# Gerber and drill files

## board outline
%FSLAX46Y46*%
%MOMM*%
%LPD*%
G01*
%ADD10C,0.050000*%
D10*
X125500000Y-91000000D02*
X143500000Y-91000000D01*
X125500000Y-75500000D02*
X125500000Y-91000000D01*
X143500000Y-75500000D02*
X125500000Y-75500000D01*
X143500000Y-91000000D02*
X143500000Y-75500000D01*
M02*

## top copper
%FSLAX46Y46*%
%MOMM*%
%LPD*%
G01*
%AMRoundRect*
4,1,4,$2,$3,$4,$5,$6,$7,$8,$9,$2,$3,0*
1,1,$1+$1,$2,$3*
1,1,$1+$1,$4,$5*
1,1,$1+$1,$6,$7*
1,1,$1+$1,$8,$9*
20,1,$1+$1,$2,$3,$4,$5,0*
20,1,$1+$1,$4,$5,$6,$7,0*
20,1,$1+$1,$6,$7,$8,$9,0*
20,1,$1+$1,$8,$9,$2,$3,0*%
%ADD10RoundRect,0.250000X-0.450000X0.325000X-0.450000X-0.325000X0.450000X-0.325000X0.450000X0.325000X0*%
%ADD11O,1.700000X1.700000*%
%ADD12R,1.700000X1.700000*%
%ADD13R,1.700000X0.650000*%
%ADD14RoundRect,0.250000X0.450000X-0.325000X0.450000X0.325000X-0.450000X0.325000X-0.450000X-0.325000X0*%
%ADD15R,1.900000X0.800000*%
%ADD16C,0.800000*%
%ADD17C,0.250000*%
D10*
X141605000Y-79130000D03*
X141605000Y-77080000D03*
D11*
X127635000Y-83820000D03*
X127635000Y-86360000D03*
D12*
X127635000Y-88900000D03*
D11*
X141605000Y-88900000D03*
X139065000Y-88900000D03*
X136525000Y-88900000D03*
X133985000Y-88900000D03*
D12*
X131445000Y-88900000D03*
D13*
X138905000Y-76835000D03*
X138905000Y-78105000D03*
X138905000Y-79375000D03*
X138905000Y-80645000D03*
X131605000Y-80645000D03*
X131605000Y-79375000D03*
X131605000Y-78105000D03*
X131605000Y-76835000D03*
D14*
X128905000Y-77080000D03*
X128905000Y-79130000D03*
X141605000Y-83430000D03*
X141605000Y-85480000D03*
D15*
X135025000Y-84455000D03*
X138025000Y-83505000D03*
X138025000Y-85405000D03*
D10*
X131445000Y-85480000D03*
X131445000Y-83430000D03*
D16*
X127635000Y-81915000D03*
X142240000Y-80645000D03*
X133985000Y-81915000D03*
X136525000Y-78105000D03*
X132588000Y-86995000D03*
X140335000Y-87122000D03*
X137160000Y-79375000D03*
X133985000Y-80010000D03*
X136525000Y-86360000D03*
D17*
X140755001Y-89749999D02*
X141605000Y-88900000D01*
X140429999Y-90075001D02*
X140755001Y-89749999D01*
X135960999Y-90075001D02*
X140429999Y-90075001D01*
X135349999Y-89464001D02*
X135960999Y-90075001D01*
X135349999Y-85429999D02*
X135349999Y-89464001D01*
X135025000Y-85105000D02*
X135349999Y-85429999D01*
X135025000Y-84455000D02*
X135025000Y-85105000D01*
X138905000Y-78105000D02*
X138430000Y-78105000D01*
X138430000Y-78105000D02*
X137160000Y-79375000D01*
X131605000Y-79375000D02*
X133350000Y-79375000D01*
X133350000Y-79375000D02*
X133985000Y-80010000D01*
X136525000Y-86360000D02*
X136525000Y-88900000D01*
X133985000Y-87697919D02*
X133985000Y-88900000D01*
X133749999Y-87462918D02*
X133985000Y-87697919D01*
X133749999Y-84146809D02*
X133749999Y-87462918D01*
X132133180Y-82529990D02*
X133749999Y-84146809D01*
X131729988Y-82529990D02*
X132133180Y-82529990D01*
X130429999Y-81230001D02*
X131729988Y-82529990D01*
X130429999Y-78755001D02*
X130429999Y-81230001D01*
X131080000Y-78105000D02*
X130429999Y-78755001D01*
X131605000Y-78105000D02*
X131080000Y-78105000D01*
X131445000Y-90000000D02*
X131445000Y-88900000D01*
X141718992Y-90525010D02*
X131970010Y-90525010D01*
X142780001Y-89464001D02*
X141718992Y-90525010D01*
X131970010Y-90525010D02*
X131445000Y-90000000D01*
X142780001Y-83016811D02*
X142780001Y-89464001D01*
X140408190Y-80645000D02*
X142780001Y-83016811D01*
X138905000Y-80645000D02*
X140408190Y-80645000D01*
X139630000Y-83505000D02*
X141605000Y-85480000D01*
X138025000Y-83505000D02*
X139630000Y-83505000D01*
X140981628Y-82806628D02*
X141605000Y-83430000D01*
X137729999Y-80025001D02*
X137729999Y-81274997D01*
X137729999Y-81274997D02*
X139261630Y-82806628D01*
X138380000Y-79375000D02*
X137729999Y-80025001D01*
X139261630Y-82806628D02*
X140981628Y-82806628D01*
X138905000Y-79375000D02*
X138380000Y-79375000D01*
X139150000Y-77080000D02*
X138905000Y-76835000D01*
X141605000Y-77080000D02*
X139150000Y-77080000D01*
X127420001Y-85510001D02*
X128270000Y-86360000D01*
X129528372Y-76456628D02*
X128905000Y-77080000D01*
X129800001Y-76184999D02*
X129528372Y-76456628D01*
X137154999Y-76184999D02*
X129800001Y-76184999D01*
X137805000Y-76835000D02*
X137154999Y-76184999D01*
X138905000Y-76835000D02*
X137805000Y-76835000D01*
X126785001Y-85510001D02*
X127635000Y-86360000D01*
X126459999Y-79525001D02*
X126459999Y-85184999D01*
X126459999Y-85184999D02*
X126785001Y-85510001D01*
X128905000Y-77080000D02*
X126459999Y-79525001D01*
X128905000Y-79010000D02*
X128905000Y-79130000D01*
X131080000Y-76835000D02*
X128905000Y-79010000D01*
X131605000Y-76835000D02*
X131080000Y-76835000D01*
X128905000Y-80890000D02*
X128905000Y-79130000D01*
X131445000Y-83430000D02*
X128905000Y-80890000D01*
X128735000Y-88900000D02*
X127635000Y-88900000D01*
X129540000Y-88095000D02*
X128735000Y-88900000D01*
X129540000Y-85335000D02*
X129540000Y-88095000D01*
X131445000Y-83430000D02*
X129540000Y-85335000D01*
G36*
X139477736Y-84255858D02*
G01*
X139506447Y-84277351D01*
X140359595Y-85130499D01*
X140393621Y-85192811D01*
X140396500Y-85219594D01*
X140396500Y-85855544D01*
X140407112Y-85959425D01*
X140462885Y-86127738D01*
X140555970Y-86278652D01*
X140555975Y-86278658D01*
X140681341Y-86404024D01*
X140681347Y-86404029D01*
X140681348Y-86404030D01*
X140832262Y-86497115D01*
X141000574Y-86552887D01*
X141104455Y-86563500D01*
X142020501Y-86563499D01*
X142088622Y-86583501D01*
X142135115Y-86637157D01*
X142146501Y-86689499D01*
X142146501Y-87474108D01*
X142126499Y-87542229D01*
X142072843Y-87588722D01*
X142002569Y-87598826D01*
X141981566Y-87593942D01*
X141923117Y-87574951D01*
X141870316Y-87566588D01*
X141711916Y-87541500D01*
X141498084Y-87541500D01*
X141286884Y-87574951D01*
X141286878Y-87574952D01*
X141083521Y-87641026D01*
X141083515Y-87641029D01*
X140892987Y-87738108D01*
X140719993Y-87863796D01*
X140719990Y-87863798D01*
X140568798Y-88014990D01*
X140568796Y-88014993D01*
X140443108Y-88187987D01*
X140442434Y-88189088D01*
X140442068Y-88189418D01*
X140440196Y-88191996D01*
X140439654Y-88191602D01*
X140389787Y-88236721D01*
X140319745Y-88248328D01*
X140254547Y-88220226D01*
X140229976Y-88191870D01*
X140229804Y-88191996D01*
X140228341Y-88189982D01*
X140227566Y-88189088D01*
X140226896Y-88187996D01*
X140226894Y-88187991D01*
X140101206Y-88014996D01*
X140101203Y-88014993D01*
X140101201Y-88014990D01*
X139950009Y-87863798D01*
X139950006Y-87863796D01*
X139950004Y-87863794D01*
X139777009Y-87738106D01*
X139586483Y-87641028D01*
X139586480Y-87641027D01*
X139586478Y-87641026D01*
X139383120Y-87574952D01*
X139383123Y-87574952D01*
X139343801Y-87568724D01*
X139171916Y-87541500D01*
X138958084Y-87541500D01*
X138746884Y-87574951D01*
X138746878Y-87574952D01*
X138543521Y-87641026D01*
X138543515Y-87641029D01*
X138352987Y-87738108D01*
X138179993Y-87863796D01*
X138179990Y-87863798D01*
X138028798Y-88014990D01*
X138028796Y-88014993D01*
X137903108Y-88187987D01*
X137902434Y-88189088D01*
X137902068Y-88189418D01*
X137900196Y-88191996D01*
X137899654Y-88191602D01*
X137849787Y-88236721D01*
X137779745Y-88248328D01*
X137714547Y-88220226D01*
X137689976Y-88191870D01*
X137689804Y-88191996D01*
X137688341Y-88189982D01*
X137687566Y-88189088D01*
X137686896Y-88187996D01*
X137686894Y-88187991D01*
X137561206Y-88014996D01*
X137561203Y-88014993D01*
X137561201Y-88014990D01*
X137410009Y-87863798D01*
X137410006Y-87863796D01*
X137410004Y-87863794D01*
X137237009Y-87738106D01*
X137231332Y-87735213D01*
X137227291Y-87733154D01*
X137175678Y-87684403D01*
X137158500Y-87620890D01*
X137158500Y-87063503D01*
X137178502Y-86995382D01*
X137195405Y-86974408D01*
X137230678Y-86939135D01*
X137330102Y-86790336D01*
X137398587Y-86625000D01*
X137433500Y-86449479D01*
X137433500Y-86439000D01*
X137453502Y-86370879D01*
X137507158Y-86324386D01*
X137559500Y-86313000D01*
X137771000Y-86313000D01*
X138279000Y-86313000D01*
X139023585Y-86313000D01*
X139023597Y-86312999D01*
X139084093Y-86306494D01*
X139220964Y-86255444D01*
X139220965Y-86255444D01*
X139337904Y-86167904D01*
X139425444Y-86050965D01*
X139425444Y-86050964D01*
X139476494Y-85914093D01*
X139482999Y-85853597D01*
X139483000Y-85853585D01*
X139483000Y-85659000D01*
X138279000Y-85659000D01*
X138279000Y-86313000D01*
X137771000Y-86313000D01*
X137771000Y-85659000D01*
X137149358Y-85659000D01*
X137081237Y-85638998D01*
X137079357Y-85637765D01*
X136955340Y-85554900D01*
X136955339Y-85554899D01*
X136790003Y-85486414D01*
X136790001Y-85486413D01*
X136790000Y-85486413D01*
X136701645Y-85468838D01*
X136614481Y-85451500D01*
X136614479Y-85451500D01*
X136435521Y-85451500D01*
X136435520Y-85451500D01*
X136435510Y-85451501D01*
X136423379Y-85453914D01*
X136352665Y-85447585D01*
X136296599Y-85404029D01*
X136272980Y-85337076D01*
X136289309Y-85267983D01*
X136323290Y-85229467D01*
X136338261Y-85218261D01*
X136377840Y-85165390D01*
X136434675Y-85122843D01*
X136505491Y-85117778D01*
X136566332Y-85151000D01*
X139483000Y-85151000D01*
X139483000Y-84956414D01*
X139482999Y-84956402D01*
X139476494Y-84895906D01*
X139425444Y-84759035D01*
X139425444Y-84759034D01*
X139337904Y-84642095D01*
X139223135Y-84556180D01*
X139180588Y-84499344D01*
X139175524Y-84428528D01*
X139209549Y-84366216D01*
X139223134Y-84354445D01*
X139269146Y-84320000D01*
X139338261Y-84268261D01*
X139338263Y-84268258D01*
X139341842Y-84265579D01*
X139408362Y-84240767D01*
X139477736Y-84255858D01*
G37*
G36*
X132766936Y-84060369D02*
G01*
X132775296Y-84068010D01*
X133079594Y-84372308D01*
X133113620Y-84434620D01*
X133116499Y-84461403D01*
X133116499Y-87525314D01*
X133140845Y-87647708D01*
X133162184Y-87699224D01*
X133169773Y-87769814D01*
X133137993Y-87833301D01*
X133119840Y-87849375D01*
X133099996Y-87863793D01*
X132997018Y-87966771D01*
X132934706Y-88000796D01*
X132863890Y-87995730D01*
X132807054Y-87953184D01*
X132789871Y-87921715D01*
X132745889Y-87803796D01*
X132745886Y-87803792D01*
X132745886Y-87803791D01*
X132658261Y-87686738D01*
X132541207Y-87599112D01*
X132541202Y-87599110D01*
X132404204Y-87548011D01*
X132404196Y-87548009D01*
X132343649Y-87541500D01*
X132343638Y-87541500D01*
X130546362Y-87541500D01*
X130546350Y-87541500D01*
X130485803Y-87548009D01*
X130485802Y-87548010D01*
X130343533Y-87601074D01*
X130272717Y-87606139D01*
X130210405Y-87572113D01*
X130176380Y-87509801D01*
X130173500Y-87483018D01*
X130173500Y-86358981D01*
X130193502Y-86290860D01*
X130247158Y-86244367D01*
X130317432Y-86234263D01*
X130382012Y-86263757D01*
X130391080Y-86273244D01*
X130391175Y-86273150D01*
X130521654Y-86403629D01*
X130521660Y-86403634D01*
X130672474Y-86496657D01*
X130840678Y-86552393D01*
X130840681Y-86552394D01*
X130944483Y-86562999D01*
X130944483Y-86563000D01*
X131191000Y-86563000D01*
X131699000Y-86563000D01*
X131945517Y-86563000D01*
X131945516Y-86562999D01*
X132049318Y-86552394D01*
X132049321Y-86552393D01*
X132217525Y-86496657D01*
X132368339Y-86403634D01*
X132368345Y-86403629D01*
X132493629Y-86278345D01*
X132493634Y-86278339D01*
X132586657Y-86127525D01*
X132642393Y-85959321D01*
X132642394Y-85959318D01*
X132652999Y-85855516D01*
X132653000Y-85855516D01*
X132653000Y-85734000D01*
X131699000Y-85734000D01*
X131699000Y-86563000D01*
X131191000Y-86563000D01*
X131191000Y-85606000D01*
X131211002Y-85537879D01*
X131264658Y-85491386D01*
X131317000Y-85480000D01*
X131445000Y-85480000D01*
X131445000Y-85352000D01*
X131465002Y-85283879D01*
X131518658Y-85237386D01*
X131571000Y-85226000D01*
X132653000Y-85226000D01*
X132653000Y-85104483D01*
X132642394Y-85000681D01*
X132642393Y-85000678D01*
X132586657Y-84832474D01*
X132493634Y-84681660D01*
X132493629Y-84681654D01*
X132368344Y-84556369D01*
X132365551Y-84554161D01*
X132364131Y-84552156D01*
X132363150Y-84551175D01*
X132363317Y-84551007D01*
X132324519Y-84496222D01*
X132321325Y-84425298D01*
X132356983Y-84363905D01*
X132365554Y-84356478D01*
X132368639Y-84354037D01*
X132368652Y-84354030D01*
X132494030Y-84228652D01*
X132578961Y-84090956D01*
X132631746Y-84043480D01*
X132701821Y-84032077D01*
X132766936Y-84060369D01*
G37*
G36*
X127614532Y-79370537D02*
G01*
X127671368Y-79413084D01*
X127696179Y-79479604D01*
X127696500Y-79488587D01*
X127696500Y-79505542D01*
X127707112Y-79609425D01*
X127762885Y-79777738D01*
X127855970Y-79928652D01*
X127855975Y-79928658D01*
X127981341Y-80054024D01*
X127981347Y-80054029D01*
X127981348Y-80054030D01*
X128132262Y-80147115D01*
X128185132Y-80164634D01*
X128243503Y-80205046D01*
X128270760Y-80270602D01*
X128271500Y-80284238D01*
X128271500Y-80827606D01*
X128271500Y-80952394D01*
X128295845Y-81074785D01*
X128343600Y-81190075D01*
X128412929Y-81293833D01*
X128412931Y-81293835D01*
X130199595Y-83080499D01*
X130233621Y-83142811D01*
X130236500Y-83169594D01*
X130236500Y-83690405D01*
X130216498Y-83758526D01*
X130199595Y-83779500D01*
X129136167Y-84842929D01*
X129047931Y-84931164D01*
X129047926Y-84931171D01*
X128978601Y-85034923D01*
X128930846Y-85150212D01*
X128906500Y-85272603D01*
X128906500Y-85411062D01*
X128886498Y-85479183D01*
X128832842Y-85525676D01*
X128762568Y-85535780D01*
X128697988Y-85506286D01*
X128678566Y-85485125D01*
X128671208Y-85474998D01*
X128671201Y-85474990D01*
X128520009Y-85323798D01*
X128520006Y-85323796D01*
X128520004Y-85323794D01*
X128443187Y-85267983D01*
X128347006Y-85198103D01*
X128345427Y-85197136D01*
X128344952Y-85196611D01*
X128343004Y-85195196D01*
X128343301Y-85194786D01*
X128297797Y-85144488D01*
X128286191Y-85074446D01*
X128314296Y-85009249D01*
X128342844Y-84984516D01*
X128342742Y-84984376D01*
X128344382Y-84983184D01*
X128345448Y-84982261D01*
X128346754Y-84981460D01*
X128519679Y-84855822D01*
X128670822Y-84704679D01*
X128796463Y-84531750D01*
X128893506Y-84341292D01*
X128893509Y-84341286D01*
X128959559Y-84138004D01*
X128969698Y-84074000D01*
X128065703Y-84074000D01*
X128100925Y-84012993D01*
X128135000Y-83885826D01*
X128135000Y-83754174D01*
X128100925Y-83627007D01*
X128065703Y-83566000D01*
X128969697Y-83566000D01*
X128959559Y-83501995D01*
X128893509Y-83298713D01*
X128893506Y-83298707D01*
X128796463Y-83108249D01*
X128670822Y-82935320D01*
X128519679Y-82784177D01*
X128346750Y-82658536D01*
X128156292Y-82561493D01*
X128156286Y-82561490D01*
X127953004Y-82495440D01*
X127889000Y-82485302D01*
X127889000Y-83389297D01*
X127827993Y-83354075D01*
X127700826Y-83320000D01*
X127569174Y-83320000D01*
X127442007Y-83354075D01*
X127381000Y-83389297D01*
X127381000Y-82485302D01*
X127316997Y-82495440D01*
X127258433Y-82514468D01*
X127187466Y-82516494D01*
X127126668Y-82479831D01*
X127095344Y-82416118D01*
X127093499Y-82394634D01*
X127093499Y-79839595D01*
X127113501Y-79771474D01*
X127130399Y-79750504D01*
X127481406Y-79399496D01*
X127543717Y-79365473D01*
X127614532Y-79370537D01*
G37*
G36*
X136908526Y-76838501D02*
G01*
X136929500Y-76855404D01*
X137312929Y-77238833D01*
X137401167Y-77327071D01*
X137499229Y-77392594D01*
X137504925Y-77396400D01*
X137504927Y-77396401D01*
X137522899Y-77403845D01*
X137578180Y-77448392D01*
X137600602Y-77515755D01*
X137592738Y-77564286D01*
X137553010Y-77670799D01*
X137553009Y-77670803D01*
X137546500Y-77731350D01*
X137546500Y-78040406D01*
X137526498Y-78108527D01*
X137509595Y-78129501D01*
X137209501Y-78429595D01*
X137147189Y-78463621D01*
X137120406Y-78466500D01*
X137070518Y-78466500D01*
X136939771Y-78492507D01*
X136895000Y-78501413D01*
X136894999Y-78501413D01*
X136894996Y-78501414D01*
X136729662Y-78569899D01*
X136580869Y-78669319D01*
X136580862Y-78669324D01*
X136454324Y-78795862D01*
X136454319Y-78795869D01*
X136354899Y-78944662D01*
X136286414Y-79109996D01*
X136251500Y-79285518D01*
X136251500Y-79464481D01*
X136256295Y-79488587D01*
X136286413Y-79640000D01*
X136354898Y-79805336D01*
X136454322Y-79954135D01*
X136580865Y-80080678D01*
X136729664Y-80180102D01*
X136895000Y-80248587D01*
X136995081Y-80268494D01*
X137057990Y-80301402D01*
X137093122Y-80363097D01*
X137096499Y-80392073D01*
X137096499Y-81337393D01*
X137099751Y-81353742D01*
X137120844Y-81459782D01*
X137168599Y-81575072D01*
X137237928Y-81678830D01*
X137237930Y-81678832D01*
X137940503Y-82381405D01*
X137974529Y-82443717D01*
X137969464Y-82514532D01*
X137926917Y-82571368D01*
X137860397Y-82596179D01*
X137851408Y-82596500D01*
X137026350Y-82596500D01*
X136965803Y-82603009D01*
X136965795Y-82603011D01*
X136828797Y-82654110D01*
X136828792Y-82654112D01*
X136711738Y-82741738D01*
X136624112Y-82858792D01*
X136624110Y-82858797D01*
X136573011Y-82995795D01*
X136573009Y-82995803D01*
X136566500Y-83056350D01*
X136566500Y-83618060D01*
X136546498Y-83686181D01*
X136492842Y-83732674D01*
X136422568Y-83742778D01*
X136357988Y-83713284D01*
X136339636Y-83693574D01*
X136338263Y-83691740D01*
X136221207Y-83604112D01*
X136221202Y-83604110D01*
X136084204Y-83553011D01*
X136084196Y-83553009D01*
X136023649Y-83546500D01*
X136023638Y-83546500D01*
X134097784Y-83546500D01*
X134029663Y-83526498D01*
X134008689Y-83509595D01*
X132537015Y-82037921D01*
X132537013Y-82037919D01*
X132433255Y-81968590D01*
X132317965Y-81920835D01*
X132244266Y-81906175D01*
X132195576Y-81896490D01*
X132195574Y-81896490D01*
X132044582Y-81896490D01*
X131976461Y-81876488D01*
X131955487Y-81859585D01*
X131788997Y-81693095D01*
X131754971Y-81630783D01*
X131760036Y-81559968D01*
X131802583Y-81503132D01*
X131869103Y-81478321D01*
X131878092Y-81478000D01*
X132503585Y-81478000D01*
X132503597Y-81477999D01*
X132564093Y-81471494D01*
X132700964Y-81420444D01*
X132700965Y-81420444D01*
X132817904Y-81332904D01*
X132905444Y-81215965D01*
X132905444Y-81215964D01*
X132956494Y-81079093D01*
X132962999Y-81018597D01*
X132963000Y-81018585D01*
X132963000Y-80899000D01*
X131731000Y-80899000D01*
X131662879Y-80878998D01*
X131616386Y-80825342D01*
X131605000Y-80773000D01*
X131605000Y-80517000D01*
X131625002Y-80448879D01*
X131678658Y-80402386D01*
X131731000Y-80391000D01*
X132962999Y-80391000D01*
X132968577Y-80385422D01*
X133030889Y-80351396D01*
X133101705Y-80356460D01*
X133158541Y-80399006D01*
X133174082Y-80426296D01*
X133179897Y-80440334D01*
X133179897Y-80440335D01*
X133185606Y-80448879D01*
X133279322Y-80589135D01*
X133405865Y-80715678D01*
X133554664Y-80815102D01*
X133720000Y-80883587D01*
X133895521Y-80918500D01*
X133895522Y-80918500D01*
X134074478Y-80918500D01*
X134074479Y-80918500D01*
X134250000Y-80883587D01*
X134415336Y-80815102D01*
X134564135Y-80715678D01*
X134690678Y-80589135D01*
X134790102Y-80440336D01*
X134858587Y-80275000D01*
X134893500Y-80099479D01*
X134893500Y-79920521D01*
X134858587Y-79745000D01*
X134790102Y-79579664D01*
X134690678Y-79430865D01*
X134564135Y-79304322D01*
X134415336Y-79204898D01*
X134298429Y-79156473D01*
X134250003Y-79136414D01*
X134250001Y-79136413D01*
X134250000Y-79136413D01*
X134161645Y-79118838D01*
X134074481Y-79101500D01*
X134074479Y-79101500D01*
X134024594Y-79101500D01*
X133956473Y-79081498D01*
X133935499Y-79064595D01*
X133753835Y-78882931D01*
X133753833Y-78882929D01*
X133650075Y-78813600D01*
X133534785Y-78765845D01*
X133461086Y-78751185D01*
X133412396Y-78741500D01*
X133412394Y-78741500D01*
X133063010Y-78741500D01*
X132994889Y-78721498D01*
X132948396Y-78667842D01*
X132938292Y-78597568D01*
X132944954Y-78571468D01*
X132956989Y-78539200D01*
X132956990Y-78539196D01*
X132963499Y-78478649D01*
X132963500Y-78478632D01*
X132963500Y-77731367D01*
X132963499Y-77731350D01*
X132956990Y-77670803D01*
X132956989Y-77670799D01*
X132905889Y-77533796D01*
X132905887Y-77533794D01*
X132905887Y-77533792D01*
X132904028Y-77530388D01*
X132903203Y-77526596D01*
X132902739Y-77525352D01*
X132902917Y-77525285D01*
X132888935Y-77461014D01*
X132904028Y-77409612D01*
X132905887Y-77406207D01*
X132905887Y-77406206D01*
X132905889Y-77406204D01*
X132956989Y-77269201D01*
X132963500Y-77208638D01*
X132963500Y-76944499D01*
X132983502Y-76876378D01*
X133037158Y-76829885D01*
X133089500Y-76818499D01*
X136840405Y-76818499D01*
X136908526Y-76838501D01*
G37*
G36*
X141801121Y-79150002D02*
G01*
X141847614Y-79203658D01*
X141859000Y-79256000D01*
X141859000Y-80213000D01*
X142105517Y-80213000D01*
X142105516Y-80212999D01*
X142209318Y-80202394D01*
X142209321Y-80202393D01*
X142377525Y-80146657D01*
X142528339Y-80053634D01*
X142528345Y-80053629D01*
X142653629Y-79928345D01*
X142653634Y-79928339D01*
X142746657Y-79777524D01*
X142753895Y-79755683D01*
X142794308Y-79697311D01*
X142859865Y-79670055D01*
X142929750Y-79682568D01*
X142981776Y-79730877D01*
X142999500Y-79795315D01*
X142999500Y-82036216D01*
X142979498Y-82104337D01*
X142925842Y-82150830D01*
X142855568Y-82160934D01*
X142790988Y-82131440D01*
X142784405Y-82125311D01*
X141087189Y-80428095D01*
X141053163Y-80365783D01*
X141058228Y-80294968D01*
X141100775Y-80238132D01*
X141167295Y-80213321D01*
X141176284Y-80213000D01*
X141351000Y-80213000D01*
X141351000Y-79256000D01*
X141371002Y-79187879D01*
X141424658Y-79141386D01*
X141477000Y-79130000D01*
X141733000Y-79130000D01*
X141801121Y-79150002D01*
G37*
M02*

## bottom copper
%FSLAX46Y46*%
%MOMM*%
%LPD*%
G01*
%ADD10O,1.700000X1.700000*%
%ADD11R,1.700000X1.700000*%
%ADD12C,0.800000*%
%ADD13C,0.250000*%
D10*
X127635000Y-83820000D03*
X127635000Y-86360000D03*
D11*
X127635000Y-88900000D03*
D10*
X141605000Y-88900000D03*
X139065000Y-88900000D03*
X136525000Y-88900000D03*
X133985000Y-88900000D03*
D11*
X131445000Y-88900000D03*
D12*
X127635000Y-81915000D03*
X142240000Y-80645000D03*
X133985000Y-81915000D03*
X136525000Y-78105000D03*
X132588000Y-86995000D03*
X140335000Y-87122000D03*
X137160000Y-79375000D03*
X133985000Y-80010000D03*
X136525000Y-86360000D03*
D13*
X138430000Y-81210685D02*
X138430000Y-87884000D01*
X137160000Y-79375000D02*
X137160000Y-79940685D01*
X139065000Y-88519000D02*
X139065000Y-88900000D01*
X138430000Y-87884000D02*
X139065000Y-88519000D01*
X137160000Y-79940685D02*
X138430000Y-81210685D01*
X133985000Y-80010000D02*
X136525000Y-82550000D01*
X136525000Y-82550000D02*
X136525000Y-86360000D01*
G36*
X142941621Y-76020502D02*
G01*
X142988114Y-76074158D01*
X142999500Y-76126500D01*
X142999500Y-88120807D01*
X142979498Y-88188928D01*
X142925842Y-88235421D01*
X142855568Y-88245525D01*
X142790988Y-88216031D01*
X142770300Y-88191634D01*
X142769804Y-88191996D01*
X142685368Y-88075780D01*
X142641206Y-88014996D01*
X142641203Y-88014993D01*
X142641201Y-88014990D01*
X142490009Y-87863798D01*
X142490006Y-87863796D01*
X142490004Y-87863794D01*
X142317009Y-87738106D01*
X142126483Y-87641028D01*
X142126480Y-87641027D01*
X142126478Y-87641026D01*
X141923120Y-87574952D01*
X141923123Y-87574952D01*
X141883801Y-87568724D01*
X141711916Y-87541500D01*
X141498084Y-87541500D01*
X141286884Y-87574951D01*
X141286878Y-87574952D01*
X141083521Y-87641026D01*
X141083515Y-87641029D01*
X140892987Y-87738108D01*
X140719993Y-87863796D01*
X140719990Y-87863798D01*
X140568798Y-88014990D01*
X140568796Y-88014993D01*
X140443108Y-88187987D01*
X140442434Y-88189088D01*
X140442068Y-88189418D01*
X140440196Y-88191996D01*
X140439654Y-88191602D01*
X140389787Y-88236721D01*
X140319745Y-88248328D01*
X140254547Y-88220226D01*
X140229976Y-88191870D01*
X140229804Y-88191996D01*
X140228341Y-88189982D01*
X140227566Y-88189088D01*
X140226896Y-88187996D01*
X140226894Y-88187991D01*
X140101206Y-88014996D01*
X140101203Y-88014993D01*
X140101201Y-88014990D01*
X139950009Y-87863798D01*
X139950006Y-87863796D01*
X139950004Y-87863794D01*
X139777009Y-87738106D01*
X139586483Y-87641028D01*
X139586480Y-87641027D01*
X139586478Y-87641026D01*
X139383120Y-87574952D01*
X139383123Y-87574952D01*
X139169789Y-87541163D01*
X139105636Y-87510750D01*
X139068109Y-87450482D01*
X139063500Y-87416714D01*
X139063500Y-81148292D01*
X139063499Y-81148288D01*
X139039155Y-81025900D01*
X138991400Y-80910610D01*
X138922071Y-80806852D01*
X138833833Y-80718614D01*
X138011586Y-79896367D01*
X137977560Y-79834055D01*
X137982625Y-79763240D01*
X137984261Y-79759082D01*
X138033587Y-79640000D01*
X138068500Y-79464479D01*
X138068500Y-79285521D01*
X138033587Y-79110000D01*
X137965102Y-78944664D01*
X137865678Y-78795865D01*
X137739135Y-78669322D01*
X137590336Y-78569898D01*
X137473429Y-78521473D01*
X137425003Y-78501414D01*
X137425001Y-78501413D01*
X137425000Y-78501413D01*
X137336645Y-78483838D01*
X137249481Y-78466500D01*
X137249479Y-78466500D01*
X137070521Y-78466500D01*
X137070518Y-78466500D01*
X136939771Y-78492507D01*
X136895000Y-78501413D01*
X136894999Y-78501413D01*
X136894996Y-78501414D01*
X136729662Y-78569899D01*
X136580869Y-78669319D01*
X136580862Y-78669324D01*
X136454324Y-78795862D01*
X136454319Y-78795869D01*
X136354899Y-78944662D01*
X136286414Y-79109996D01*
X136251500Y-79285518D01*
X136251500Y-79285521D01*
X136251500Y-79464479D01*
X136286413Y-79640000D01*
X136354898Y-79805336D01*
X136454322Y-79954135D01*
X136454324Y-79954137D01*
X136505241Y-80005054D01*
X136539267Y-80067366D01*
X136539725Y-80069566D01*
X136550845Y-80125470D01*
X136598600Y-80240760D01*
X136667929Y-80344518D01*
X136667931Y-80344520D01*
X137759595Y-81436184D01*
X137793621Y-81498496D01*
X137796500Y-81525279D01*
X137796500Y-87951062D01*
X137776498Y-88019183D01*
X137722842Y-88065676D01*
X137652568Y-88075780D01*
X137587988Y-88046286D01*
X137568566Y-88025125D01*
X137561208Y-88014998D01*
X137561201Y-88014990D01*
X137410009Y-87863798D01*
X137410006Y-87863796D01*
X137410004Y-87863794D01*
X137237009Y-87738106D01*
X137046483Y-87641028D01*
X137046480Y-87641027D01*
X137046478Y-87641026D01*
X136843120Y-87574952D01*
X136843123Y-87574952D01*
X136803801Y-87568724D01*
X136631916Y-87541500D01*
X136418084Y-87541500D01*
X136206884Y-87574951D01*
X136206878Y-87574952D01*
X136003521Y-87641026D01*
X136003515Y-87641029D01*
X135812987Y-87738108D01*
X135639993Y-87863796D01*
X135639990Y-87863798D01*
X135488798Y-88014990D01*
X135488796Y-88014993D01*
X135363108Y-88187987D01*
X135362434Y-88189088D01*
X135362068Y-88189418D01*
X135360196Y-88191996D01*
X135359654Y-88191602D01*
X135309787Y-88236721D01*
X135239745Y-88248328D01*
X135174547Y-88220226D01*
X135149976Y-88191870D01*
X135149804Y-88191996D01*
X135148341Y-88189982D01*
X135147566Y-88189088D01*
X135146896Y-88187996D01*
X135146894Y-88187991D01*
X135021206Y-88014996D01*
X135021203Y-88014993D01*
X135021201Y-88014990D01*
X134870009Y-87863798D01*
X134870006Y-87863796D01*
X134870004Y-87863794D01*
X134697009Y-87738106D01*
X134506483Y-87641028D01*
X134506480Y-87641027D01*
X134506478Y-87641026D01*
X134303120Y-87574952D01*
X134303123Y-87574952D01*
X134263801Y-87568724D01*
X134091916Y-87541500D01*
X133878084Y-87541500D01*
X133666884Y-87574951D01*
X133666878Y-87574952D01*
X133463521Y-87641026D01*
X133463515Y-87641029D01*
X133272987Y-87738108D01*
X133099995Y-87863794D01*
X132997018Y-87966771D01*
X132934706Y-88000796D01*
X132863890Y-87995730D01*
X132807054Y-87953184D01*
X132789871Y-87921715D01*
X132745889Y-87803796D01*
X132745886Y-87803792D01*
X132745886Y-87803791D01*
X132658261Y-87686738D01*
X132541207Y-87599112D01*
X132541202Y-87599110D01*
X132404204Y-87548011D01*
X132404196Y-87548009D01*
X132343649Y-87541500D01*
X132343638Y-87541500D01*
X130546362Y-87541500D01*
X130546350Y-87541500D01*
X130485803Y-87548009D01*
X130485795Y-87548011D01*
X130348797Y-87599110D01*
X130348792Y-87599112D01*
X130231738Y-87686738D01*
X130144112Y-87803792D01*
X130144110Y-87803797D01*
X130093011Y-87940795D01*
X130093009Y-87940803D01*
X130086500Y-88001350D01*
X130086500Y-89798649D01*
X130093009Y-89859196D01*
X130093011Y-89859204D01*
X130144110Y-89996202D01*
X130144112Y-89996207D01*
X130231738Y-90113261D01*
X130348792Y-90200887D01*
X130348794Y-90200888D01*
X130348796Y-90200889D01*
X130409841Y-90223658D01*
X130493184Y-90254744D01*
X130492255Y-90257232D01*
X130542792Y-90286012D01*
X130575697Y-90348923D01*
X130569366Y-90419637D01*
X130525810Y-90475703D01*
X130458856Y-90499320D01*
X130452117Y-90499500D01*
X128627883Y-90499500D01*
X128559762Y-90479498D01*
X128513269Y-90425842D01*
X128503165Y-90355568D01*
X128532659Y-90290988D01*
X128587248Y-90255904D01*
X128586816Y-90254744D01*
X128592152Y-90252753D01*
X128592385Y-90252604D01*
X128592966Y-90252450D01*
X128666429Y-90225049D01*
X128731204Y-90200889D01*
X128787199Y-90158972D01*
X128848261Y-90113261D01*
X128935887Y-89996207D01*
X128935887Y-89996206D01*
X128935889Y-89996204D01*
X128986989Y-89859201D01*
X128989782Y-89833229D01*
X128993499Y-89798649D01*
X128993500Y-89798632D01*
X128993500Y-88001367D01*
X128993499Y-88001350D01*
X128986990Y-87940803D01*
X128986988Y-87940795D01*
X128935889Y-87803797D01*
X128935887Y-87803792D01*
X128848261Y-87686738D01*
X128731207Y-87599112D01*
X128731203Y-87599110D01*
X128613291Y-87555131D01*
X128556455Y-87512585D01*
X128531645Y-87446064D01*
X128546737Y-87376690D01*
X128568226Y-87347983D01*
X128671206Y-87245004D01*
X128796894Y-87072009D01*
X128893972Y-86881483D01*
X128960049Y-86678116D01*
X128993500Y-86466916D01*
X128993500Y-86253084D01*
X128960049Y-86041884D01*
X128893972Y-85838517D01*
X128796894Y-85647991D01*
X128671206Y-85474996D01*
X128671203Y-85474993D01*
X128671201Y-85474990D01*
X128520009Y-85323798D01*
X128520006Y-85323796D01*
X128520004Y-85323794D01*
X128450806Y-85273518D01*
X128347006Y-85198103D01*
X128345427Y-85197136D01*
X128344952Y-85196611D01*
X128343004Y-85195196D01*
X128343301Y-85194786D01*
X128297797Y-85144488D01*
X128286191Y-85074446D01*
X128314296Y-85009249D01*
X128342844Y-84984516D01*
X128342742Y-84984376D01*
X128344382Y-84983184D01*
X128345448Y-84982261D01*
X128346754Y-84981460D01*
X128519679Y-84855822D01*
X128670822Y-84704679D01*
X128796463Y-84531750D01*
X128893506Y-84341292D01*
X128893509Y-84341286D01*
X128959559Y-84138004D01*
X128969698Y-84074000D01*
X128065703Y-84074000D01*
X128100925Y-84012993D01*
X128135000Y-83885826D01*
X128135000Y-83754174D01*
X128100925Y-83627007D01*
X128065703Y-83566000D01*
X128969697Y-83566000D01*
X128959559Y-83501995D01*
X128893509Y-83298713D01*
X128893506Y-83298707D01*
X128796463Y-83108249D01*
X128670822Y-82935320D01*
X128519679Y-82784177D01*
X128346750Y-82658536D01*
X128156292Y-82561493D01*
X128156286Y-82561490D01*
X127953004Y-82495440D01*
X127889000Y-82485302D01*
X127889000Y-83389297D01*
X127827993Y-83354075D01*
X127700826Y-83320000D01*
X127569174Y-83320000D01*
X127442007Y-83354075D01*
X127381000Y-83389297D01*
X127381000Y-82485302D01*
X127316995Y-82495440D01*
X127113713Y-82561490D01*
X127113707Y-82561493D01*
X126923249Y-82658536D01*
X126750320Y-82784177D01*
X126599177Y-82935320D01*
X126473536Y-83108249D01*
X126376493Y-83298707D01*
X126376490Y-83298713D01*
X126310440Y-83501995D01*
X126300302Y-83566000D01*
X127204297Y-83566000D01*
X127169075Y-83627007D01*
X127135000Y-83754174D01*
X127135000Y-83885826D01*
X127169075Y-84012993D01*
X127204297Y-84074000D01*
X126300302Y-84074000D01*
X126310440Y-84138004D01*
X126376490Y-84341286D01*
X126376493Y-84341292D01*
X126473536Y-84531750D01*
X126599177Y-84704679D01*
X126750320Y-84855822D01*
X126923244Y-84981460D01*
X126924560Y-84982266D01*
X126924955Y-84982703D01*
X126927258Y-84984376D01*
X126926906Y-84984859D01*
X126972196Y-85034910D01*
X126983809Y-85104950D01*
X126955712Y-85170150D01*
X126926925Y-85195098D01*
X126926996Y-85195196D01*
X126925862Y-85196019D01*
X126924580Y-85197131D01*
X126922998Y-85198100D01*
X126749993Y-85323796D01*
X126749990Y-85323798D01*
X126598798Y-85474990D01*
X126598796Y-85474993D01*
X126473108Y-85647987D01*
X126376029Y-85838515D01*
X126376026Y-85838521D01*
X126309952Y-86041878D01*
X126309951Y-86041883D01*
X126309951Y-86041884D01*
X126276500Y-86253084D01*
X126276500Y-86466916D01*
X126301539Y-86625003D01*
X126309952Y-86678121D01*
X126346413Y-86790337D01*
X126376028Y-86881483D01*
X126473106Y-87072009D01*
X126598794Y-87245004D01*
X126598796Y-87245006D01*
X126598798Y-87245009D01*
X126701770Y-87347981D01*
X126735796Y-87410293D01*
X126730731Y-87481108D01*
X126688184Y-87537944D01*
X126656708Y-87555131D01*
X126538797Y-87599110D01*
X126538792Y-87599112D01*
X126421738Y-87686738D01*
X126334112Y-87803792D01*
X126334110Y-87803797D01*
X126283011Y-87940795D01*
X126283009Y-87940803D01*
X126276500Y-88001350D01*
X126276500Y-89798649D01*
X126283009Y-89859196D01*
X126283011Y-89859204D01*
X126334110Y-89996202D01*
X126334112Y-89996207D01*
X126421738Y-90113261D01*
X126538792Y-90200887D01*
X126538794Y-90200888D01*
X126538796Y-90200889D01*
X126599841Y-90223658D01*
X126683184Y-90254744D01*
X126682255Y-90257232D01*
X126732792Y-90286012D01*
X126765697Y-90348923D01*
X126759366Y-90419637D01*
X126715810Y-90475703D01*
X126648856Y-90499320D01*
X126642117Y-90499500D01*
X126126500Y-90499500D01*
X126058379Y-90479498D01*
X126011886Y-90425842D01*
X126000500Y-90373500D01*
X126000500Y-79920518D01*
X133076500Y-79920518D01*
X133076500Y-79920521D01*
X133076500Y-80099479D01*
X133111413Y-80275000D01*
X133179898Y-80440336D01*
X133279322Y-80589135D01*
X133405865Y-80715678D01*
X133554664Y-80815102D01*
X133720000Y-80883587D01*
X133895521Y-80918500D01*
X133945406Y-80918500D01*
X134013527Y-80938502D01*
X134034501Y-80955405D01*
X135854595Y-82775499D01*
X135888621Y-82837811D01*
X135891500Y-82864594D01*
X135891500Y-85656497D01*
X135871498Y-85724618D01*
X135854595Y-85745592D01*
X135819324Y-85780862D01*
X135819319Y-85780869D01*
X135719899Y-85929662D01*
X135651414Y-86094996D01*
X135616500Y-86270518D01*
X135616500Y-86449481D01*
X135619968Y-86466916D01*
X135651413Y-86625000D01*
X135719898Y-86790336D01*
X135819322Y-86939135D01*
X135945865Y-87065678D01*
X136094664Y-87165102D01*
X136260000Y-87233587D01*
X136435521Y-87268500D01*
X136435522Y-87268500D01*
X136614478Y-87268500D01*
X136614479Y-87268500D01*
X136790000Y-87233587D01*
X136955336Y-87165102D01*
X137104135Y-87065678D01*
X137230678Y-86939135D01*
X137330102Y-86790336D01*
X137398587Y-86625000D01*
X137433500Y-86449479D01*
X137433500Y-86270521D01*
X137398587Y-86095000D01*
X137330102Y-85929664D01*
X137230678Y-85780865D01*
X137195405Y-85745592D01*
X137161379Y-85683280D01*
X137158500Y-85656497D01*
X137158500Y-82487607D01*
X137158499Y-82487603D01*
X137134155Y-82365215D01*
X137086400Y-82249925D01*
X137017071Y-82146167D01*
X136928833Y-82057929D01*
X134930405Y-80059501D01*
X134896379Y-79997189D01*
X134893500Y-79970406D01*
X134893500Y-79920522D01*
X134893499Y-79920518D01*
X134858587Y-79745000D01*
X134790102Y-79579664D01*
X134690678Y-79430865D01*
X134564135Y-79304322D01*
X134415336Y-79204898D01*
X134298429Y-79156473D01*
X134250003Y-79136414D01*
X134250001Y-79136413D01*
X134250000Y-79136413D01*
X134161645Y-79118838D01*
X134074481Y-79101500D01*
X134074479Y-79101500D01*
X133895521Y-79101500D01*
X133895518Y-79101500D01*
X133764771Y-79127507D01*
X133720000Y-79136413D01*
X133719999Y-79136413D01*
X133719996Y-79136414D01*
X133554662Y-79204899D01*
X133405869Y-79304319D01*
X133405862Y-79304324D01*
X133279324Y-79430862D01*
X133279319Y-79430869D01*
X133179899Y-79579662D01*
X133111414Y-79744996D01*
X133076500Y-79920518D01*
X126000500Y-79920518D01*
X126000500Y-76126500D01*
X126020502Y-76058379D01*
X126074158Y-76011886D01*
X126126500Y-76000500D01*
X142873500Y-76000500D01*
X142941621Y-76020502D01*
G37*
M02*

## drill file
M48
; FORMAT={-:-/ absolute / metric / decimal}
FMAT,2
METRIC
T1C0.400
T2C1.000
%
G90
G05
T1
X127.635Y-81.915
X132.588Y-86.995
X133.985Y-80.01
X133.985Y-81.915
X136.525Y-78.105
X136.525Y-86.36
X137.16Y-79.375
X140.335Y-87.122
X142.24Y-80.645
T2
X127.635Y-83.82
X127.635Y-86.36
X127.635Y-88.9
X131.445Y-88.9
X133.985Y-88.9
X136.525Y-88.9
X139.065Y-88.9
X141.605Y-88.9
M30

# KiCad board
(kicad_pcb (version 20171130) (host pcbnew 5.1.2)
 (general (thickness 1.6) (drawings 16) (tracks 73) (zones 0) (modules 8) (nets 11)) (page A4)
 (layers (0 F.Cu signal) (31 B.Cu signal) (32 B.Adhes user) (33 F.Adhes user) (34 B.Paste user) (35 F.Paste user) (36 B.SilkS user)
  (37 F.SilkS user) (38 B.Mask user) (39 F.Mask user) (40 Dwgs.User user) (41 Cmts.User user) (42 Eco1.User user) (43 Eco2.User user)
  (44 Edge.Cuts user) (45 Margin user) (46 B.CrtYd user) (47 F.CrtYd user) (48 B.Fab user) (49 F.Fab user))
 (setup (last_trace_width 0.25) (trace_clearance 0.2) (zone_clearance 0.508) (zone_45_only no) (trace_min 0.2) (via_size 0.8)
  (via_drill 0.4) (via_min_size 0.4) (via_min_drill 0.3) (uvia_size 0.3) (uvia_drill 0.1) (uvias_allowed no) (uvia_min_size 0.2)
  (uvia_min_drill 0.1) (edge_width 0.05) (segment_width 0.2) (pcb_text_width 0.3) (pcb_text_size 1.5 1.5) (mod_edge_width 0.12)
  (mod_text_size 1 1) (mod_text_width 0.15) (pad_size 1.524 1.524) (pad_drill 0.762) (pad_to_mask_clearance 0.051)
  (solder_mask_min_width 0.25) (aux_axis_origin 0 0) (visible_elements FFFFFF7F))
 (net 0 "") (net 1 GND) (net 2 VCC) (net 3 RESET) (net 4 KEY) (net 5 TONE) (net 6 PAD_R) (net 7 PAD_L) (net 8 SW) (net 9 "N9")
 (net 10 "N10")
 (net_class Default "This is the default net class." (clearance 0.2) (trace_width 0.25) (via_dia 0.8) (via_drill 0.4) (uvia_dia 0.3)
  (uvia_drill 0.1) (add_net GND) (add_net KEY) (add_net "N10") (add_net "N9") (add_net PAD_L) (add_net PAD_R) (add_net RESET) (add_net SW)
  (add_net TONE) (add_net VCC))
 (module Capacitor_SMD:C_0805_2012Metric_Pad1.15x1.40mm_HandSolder (layer F.Cu) (at 141.605 78.105 270)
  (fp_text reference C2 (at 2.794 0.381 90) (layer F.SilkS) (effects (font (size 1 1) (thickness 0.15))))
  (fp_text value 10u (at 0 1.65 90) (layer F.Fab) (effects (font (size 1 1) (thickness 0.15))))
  (pad 2 smd roundrect (at 1.025 0 270) (size 1.15 1.4) (layers F.Cu F.Paste F.Mask) (roundrect_rratio 0.217391) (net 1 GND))
  (pad 1 smd roundrect (at -1.025 0 270) (size 1.15 1.4) (layers F.Cu F.Paste F.Mask) (roundrect_rratio 0.217391) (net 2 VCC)))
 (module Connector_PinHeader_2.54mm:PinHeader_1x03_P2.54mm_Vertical (layer F.Cu) (at 127.635 88.9 180)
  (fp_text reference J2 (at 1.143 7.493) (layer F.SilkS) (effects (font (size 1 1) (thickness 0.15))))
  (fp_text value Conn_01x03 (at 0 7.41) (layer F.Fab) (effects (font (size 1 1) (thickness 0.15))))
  (pad 3 thru_hole oval (at 0 5.08 180) (size 1.7 1.7) (drill 1) (layers *.Cu *.Mask) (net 1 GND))
  (pad 2 thru_hole oval (at 0 2.54 180) (size 1.7 1.7) (drill 1) (layers *.Cu *.Mask) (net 2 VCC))
  (pad 1 thru_hole rect (at 0 0 180) (size 1.7 1.7) (drill 1) (layers *.Cu *.Mask) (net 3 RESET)))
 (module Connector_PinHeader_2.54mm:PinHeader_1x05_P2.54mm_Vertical (layer F.Cu) (at 131.445 88.9 90)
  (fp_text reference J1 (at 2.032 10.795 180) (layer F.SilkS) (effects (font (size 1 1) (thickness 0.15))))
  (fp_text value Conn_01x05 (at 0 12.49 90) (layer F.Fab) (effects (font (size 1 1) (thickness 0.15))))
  (pad 5 thru_hole oval (at 0 10.16 90) (size 1.7 1.7) (drill 1) (layers *.Cu *.Mask) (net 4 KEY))
  (pad 4 thru_hole oval (at 0 7.62 90) (size 1.7 1.7) (drill 1) (layers *.Cu *.Mask) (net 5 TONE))
  (pad 3 thru_hole oval (at 0 5.08 90) (size 1.7 1.7) (drill 1) (layers *.Cu *.Mask) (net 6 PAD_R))
  (pad 2 thru_hole oval (at 0 2.54 90) (size 1.7 1.7) (drill 1) (layers *.Cu *.Mask) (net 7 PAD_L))
  (pad 1 thru_hole rect (at 0 0 90) (size 1.7 1.7) (drill 1) (layers *.Cu *.Mask) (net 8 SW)))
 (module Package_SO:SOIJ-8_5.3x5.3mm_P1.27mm (layer F.Cu) (at 135.255 78.74)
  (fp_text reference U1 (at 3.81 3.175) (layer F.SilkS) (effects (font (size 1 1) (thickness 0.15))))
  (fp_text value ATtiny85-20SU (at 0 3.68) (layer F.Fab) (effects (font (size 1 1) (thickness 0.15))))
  (pad 8 smd rect (at 3.65 -1.905) (size 1.7 0.65) (layers F.Cu F.Paste F.Mask) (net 2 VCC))
  (pad 7 smd rect (at 3.65 -0.635) (size 1.7 0.65) (layers F.Cu F.Paste F.Mask) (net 5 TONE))
  (pad 6 smd rect (at 3.65 0.635) (size 1.7 0.65) (layers F.Cu F.Paste F.Mask) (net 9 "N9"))
  (pad 5 smd rect (at 3.65 1.905) (size 1.7 0.65) (layers F.Cu F.Paste F.Mask) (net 8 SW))
  (pad 4 smd rect (at -3.65 1.905) (size 1.7 0.65) (layers F.Cu F.Paste F.Mask) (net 1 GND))
  (pad 3 smd rect (at -3.65 0.635) (size 1.7 0.65) (layers F.Cu F.Paste F.Mask) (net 6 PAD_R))
  (pad 2 smd rect (at -3.65 -0.635) (size 1.7 0.65) (layers F.Cu F.Paste F.Mask) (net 7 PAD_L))
  (pad 1 smd rect (at -3.65 -1.905) (size 1.7 0.65) (layers F.Cu F.Paste F.Mask) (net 3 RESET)))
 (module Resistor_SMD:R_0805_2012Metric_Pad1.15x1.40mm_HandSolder (layer F.Cu) (at 128.905 78.105 90)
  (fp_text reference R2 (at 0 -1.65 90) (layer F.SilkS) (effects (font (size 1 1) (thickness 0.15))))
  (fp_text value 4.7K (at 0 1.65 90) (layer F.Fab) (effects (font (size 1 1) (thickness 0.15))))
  (pad 2 smd roundrect (at 1.025 0 90) (size 1.15 1.4) (layers F.Cu F.Paste F.Mask) (roundrect_rratio 0.217391) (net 2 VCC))
  (pad 1 smd roundrect (at -1.025 0 90) (size 1.15 1.4) (layers F.Cu F.Paste F.Mask) (roundrect_rratio 0.217391) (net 3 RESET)))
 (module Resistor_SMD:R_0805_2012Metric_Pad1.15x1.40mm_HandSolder (layer F.Cu) (at 141.605 84.455 90)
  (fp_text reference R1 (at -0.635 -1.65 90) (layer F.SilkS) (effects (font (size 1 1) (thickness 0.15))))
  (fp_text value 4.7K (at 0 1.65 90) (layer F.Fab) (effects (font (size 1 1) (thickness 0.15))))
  (pad 2 smd roundrect (at 1.025 0 90) (size 1.15 1.4) (layers F.Cu F.Paste F.Mask) (roundrect_rratio 0.217391) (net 9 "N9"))
  (pad 1 smd roundrect (at -1.025 0 90) (size 1.15 1.4) (layers F.Cu F.Paste F.Mask) (roundrect_rratio 0.217391) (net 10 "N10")))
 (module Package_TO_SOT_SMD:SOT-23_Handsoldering (layer F.Cu) (at 136.525 84.455 180)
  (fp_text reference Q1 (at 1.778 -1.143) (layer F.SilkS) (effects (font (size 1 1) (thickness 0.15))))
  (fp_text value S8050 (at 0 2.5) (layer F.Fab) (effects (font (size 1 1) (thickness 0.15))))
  (pad 3 smd rect (at 1.5 0 180) (size 1.9 0.8) (layers F.Cu F.Paste F.Mask) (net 4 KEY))
  (pad 2 smd rect (at -1.5 0.95 180) (size 1.9 0.8) (layers F.Cu F.Paste F.Mask) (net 10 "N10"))
  (pad 1 smd rect (at -1.5 -0.95 180) (size 1.9 0.8) (layers F.Cu F.Paste F.Mask) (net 1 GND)))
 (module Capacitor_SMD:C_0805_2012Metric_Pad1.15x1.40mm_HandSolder (layer F.Cu) (at 131.445 84.455 270)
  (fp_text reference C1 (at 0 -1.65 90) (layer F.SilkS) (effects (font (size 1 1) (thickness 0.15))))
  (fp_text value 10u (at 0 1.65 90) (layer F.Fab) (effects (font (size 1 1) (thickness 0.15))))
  (pad 2 smd roundrect (at 1.025 0 270) (size 1.15 1.4) (layers F.Cu F.Paste F.Mask) (roundrect_rratio 0.217391) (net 1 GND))
  (pad 1 smd roundrect (at -1.025 0 270) (size 1.15 1.4) (layers F.Cu F.Paste F.Mask) (roundrect_rratio 0.217391) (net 3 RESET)))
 (gr_line (start 125.5 91) (end 143.5 91) (layer Edge.Cuts) (width 0.05))
 (gr_line (start 125.5 75.5) (end 125.5 91) (layer Edge.Cuts) (width 0.05))
 (gr_line (start 143.5 75.5) (end 125.5 75.5) (layer Edge.Cuts) (width 0.05))
 (gr_line (start 143.5 91) (end 143.5 75.5) (layer Edge.Cuts) (width 0.05))
 (via (at 127.635 81.915) (size 0.8) (drill 0.4) (layers F.Cu B.Cu) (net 1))
 (via (at 142.24 80.645) (size 0.8) (drill 0.4) (layers F.Cu B.Cu) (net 1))
 (via (at 133.985 81.915) (size 0.8) (drill 0.4) (layers F.Cu B.Cu) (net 1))
 (via (at 136.525 78.105) (size 0.8) (drill 0.4) (layers F.Cu B.Cu) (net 1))
 (via (at 132.588 86.995) (size 0.8) (drill 0.4) (layers F.Cu B.Cu) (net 1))
 (via (at 140.335 87.122) (size 0.8) (drill 0.4) (layers F.Cu B.Cu) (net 1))
 (segment (start 140.755001 89.749999) (end 141.605 88.9) (width 0.25) (layer F.Cu) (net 4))
 (segment (start 140.429999 90.075001) (end 140.755001 89.749999) (width 0.25) (layer F.Cu) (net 4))
 (segment (start 135.960999 90.075001) (end 140.429999 90.075001) (width 0.25) (layer F.Cu) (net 4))
 (segment (start 135.349999 89.464001) (end 135.960999 90.075001) (width 0.25) (layer F.Cu) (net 4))
 (segment (start 135.349999 85.429999) (end 135.349999 89.464001) (width 0.25) (layer F.Cu) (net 4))
 (segment (start 135.025 85.105) (end 135.349999 85.429999) (width 0.25) (layer F.Cu) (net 4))
 (segment (start 135.025 84.455) (end 135.025 85.105) (width 0.25) (layer F.Cu) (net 4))
 (via (at 137.16 79.375) (size 0.8) (drill 0.4) (layers F.Cu B.Cu) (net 5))
 (segment (start 138.905 78.105) (end 138.43 78.105) (width 0.25) (layer F.Cu) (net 5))
 (segment (start 138.43 78.105) (end 137.16 79.375) (width 0.25) (layer F.Cu) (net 5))
 (segment (start 138.43 81.210685) (end 138.43 87.884) (width 0.25) (layer B.Cu) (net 5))
 (segment (start 137.16 79.375) (end 137.16 79.940685) (width 0.25) (layer B.Cu) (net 5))
 (segment (start 139.065 88.519) (end 139.065 88.9) (width 0.25) (layer B.Cu) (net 5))
 (segment (start 138.43 87.884) (end 139.065 88.519) (width 0.25) (layer B.Cu) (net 5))
 (segment (start 137.16 79.940685) (end 138.43 81.210685) (width 0.25) (layer B.Cu) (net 5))
 (via (at 133.985 80.01) (size 0.8) (drill 0.4) (layers F.Cu B.Cu) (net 6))
 (segment (start 131.605 79.375) (end 133.35 79.375) (width 0.25) (layer F.Cu) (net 6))
 (segment (start 133.35 79.375) (end 133.985 80.01) (width 0.25) (layer F.Cu) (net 6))
 (segment (start 133.985 80.01) (end 136.525 82.55) (width 0.25) (layer B.Cu) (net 6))
 (via (at 136.525 86.36) (size 0.8) (drill 0.4) (layers F.Cu B.Cu) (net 6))
 (segment (start 136.525 82.55) (end 136.525 86.36) (width 0.25) (layer B.Cu) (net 6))
 (segment (start 136.525 86.36) (end 136.525 88.9) (width 0.25) (layer F.Cu) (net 6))
 (segment (start 133.985 87.697919) (end 133.985 88.9) (width 0.25) (layer F.Cu) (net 7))
 (segment (start 133.749999 87.462918) (end 133.985 87.697919) (width 0.25) (layer F.Cu) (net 7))
 (segment (start 133.749999 84.146809) (end 133.749999 87.462918) (width 0.25) (layer F.Cu) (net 7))
 (segment (start 132.13318 82.52999) (end 133.749999 84.146809) (width 0.25) (layer F.Cu) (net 7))
 (segment (start 131.729988 82.52999) (end 132.13318 82.52999) (width 0.25) (layer F.Cu) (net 7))
 (segment (start 130.429999 81.230001) (end 131.729988 82.52999) (width 0.25) (layer F.Cu) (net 7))
 (segment (start 130.429999 78.755001) (end 130.429999 81.230001) (width 0.25) (layer F.Cu) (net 7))
 (segment (start 131.08 78.105) (end 130.429999 78.755001) (width 0.25) (layer F.Cu) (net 7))
 (segment (start 131.605 78.105) (end 131.08 78.105) (width 0.25) (layer F.Cu) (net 7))
 (segment (start 131.445 90) (end 131.445 88.9) (width 0.25) (layer F.Cu) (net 8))
 (segment (start 141.718992 90.52501) (end 131.97001 90.52501) (width 0.25) (layer F.Cu) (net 8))
 (segment (start 142.780001 89.464001) (end 141.718992 90.52501) (width 0.25) (layer F.Cu) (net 8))
 (segment (start 131.97001 90.52501) (end 131.445 90) (width 0.25) (layer F.Cu) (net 8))
 (segment (start 142.780001 83.016811) (end 142.780001 89.464001) (width 0.25) (layer F.Cu) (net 8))
 (segment (start 140.40819 80.645) (end 142.780001 83.016811) (width 0.25) (layer F.Cu) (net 8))
 (segment (start 138.905 80.645) (end 140.40819 80.645) (width 0.25) (layer F.Cu) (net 8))
 (segment (start 139.63 83.505) (end 141.605 85.48) (width 0.25) (layer F.Cu) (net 10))
 (segment (start 138.025 83.505) (end 139.63 83.505) (width 0.25) (layer F.Cu) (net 10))
 (segment (start 140.981628 82.806628) (end 141.605 83.43) (width 0.25) (layer F.Cu) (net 9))
 (segment (start 137.729999 80.025001) (end 137.729999 81.274997) (width 0.25) (layer F.Cu) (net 9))
 (segment (start 137.729999 81.274997) (end 139.26163 82.806628) (width 0.25) (layer F.Cu) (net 9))
 (segment (start 138.38 79.375) (end 137.729999 80.025001) (width 0.25) (layer F.Cu) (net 9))
 (segment (start 139.26163 82.806628) (end 140.981628 82.806628) (width 0.25) (layer F.Cu) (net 9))
 (segment (start 138.905 79.375) (end 138.38 79.375) (width 0.25) (layer F.Cu) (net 9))
 (segment (start 139.15 77.08) (end 138.905 76.835) (width 0.25) (layer F.Cu) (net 2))
 (segment (start 141.605 77.08) (end 139.15 77.08) (width 0.25) (layer F.Cu) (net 2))
 (segment (start 127.420001 85.510001) (end 128.27 86.36) (width 0.25) (layer F.Cu) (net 2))
 (segment (start 129.528372 76.456628) (end 128.905 77.08) (width 0.25) (layer F.Cu) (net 2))
 (segment (start 129.800001 76.184999) (end 129.528372 76.456628) (width 0.25) (layer F.Cu) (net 2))
 (segment (start 137.154999 76.184999) (end 129.800001 76.184999) (width 0.25) (layer F.Cu) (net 2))
 (segment (start 137.805 76.835) (end 137.154999 76.184999) (width 0.25) (layer F.Cu) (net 2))
 (segment (start 138.905 76.835) (end 137.805 76.835) (width 0.25) (layer F.Cu) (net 2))
 (segment (start 126.785001 85.510001) (end 127.635 86.36) (width 0.25) (layer F.Cu) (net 2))
 (segment (start 126.459999 79.525001) (end 126.459999 85.184999) (width 0.25) (layer F.Cu) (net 2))
 (segment (start 126.459999 85.184999) (end 126.785001 85.510001) (width 0.25) (layer F.Cu) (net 2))
 (segment (start 128.905 77.08) (end 126.459999 79.525001) (width 0.25) (layer F.Cu) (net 2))
 (segment (start 128.905 79.01) (end 128.905 79.13) (width 0.25) (layer F.Cu) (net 3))
 (segment (start 131.08 76.835) (end 128.905 79.01) (width 0.25) (layer F.Cu) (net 3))
 (segment (start 131.605 76.835) (end 131.08 76.835) (width 0.25) (layer F.Cu) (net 3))
 (segment (start 128.905 80.89) (end 128.905 79.13) (width 0.25) (layer F.Cu) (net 3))
 (segment (start 131.445 83.43) (end 128.905 80.89) (width 0.25) (layer F.Cu) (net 3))
 (segment (start 128.735 88.9) (end 127.635 88.9) (width 0.25) (layer F.Cu) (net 3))
 (segment (start 129.54 88.095) (end 128.735 88.9) (width 0.25) (layer F.Cu) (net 3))
 (segment (start 129.54 85.335) (end 129.54 88.095) (width 0.25) (layer F.Cu) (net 3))
 (segment (start 131.445 83.43) (end 129.54 85.335) (width 0.25) (layer F.Cu) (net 3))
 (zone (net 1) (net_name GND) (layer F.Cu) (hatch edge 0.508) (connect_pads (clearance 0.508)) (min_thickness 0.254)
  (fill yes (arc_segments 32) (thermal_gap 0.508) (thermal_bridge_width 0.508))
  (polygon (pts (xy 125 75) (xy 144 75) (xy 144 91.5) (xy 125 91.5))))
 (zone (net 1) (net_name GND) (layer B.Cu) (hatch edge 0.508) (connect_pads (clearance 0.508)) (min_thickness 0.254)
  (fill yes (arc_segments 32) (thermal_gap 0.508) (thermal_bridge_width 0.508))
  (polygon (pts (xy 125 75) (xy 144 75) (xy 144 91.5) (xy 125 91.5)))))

